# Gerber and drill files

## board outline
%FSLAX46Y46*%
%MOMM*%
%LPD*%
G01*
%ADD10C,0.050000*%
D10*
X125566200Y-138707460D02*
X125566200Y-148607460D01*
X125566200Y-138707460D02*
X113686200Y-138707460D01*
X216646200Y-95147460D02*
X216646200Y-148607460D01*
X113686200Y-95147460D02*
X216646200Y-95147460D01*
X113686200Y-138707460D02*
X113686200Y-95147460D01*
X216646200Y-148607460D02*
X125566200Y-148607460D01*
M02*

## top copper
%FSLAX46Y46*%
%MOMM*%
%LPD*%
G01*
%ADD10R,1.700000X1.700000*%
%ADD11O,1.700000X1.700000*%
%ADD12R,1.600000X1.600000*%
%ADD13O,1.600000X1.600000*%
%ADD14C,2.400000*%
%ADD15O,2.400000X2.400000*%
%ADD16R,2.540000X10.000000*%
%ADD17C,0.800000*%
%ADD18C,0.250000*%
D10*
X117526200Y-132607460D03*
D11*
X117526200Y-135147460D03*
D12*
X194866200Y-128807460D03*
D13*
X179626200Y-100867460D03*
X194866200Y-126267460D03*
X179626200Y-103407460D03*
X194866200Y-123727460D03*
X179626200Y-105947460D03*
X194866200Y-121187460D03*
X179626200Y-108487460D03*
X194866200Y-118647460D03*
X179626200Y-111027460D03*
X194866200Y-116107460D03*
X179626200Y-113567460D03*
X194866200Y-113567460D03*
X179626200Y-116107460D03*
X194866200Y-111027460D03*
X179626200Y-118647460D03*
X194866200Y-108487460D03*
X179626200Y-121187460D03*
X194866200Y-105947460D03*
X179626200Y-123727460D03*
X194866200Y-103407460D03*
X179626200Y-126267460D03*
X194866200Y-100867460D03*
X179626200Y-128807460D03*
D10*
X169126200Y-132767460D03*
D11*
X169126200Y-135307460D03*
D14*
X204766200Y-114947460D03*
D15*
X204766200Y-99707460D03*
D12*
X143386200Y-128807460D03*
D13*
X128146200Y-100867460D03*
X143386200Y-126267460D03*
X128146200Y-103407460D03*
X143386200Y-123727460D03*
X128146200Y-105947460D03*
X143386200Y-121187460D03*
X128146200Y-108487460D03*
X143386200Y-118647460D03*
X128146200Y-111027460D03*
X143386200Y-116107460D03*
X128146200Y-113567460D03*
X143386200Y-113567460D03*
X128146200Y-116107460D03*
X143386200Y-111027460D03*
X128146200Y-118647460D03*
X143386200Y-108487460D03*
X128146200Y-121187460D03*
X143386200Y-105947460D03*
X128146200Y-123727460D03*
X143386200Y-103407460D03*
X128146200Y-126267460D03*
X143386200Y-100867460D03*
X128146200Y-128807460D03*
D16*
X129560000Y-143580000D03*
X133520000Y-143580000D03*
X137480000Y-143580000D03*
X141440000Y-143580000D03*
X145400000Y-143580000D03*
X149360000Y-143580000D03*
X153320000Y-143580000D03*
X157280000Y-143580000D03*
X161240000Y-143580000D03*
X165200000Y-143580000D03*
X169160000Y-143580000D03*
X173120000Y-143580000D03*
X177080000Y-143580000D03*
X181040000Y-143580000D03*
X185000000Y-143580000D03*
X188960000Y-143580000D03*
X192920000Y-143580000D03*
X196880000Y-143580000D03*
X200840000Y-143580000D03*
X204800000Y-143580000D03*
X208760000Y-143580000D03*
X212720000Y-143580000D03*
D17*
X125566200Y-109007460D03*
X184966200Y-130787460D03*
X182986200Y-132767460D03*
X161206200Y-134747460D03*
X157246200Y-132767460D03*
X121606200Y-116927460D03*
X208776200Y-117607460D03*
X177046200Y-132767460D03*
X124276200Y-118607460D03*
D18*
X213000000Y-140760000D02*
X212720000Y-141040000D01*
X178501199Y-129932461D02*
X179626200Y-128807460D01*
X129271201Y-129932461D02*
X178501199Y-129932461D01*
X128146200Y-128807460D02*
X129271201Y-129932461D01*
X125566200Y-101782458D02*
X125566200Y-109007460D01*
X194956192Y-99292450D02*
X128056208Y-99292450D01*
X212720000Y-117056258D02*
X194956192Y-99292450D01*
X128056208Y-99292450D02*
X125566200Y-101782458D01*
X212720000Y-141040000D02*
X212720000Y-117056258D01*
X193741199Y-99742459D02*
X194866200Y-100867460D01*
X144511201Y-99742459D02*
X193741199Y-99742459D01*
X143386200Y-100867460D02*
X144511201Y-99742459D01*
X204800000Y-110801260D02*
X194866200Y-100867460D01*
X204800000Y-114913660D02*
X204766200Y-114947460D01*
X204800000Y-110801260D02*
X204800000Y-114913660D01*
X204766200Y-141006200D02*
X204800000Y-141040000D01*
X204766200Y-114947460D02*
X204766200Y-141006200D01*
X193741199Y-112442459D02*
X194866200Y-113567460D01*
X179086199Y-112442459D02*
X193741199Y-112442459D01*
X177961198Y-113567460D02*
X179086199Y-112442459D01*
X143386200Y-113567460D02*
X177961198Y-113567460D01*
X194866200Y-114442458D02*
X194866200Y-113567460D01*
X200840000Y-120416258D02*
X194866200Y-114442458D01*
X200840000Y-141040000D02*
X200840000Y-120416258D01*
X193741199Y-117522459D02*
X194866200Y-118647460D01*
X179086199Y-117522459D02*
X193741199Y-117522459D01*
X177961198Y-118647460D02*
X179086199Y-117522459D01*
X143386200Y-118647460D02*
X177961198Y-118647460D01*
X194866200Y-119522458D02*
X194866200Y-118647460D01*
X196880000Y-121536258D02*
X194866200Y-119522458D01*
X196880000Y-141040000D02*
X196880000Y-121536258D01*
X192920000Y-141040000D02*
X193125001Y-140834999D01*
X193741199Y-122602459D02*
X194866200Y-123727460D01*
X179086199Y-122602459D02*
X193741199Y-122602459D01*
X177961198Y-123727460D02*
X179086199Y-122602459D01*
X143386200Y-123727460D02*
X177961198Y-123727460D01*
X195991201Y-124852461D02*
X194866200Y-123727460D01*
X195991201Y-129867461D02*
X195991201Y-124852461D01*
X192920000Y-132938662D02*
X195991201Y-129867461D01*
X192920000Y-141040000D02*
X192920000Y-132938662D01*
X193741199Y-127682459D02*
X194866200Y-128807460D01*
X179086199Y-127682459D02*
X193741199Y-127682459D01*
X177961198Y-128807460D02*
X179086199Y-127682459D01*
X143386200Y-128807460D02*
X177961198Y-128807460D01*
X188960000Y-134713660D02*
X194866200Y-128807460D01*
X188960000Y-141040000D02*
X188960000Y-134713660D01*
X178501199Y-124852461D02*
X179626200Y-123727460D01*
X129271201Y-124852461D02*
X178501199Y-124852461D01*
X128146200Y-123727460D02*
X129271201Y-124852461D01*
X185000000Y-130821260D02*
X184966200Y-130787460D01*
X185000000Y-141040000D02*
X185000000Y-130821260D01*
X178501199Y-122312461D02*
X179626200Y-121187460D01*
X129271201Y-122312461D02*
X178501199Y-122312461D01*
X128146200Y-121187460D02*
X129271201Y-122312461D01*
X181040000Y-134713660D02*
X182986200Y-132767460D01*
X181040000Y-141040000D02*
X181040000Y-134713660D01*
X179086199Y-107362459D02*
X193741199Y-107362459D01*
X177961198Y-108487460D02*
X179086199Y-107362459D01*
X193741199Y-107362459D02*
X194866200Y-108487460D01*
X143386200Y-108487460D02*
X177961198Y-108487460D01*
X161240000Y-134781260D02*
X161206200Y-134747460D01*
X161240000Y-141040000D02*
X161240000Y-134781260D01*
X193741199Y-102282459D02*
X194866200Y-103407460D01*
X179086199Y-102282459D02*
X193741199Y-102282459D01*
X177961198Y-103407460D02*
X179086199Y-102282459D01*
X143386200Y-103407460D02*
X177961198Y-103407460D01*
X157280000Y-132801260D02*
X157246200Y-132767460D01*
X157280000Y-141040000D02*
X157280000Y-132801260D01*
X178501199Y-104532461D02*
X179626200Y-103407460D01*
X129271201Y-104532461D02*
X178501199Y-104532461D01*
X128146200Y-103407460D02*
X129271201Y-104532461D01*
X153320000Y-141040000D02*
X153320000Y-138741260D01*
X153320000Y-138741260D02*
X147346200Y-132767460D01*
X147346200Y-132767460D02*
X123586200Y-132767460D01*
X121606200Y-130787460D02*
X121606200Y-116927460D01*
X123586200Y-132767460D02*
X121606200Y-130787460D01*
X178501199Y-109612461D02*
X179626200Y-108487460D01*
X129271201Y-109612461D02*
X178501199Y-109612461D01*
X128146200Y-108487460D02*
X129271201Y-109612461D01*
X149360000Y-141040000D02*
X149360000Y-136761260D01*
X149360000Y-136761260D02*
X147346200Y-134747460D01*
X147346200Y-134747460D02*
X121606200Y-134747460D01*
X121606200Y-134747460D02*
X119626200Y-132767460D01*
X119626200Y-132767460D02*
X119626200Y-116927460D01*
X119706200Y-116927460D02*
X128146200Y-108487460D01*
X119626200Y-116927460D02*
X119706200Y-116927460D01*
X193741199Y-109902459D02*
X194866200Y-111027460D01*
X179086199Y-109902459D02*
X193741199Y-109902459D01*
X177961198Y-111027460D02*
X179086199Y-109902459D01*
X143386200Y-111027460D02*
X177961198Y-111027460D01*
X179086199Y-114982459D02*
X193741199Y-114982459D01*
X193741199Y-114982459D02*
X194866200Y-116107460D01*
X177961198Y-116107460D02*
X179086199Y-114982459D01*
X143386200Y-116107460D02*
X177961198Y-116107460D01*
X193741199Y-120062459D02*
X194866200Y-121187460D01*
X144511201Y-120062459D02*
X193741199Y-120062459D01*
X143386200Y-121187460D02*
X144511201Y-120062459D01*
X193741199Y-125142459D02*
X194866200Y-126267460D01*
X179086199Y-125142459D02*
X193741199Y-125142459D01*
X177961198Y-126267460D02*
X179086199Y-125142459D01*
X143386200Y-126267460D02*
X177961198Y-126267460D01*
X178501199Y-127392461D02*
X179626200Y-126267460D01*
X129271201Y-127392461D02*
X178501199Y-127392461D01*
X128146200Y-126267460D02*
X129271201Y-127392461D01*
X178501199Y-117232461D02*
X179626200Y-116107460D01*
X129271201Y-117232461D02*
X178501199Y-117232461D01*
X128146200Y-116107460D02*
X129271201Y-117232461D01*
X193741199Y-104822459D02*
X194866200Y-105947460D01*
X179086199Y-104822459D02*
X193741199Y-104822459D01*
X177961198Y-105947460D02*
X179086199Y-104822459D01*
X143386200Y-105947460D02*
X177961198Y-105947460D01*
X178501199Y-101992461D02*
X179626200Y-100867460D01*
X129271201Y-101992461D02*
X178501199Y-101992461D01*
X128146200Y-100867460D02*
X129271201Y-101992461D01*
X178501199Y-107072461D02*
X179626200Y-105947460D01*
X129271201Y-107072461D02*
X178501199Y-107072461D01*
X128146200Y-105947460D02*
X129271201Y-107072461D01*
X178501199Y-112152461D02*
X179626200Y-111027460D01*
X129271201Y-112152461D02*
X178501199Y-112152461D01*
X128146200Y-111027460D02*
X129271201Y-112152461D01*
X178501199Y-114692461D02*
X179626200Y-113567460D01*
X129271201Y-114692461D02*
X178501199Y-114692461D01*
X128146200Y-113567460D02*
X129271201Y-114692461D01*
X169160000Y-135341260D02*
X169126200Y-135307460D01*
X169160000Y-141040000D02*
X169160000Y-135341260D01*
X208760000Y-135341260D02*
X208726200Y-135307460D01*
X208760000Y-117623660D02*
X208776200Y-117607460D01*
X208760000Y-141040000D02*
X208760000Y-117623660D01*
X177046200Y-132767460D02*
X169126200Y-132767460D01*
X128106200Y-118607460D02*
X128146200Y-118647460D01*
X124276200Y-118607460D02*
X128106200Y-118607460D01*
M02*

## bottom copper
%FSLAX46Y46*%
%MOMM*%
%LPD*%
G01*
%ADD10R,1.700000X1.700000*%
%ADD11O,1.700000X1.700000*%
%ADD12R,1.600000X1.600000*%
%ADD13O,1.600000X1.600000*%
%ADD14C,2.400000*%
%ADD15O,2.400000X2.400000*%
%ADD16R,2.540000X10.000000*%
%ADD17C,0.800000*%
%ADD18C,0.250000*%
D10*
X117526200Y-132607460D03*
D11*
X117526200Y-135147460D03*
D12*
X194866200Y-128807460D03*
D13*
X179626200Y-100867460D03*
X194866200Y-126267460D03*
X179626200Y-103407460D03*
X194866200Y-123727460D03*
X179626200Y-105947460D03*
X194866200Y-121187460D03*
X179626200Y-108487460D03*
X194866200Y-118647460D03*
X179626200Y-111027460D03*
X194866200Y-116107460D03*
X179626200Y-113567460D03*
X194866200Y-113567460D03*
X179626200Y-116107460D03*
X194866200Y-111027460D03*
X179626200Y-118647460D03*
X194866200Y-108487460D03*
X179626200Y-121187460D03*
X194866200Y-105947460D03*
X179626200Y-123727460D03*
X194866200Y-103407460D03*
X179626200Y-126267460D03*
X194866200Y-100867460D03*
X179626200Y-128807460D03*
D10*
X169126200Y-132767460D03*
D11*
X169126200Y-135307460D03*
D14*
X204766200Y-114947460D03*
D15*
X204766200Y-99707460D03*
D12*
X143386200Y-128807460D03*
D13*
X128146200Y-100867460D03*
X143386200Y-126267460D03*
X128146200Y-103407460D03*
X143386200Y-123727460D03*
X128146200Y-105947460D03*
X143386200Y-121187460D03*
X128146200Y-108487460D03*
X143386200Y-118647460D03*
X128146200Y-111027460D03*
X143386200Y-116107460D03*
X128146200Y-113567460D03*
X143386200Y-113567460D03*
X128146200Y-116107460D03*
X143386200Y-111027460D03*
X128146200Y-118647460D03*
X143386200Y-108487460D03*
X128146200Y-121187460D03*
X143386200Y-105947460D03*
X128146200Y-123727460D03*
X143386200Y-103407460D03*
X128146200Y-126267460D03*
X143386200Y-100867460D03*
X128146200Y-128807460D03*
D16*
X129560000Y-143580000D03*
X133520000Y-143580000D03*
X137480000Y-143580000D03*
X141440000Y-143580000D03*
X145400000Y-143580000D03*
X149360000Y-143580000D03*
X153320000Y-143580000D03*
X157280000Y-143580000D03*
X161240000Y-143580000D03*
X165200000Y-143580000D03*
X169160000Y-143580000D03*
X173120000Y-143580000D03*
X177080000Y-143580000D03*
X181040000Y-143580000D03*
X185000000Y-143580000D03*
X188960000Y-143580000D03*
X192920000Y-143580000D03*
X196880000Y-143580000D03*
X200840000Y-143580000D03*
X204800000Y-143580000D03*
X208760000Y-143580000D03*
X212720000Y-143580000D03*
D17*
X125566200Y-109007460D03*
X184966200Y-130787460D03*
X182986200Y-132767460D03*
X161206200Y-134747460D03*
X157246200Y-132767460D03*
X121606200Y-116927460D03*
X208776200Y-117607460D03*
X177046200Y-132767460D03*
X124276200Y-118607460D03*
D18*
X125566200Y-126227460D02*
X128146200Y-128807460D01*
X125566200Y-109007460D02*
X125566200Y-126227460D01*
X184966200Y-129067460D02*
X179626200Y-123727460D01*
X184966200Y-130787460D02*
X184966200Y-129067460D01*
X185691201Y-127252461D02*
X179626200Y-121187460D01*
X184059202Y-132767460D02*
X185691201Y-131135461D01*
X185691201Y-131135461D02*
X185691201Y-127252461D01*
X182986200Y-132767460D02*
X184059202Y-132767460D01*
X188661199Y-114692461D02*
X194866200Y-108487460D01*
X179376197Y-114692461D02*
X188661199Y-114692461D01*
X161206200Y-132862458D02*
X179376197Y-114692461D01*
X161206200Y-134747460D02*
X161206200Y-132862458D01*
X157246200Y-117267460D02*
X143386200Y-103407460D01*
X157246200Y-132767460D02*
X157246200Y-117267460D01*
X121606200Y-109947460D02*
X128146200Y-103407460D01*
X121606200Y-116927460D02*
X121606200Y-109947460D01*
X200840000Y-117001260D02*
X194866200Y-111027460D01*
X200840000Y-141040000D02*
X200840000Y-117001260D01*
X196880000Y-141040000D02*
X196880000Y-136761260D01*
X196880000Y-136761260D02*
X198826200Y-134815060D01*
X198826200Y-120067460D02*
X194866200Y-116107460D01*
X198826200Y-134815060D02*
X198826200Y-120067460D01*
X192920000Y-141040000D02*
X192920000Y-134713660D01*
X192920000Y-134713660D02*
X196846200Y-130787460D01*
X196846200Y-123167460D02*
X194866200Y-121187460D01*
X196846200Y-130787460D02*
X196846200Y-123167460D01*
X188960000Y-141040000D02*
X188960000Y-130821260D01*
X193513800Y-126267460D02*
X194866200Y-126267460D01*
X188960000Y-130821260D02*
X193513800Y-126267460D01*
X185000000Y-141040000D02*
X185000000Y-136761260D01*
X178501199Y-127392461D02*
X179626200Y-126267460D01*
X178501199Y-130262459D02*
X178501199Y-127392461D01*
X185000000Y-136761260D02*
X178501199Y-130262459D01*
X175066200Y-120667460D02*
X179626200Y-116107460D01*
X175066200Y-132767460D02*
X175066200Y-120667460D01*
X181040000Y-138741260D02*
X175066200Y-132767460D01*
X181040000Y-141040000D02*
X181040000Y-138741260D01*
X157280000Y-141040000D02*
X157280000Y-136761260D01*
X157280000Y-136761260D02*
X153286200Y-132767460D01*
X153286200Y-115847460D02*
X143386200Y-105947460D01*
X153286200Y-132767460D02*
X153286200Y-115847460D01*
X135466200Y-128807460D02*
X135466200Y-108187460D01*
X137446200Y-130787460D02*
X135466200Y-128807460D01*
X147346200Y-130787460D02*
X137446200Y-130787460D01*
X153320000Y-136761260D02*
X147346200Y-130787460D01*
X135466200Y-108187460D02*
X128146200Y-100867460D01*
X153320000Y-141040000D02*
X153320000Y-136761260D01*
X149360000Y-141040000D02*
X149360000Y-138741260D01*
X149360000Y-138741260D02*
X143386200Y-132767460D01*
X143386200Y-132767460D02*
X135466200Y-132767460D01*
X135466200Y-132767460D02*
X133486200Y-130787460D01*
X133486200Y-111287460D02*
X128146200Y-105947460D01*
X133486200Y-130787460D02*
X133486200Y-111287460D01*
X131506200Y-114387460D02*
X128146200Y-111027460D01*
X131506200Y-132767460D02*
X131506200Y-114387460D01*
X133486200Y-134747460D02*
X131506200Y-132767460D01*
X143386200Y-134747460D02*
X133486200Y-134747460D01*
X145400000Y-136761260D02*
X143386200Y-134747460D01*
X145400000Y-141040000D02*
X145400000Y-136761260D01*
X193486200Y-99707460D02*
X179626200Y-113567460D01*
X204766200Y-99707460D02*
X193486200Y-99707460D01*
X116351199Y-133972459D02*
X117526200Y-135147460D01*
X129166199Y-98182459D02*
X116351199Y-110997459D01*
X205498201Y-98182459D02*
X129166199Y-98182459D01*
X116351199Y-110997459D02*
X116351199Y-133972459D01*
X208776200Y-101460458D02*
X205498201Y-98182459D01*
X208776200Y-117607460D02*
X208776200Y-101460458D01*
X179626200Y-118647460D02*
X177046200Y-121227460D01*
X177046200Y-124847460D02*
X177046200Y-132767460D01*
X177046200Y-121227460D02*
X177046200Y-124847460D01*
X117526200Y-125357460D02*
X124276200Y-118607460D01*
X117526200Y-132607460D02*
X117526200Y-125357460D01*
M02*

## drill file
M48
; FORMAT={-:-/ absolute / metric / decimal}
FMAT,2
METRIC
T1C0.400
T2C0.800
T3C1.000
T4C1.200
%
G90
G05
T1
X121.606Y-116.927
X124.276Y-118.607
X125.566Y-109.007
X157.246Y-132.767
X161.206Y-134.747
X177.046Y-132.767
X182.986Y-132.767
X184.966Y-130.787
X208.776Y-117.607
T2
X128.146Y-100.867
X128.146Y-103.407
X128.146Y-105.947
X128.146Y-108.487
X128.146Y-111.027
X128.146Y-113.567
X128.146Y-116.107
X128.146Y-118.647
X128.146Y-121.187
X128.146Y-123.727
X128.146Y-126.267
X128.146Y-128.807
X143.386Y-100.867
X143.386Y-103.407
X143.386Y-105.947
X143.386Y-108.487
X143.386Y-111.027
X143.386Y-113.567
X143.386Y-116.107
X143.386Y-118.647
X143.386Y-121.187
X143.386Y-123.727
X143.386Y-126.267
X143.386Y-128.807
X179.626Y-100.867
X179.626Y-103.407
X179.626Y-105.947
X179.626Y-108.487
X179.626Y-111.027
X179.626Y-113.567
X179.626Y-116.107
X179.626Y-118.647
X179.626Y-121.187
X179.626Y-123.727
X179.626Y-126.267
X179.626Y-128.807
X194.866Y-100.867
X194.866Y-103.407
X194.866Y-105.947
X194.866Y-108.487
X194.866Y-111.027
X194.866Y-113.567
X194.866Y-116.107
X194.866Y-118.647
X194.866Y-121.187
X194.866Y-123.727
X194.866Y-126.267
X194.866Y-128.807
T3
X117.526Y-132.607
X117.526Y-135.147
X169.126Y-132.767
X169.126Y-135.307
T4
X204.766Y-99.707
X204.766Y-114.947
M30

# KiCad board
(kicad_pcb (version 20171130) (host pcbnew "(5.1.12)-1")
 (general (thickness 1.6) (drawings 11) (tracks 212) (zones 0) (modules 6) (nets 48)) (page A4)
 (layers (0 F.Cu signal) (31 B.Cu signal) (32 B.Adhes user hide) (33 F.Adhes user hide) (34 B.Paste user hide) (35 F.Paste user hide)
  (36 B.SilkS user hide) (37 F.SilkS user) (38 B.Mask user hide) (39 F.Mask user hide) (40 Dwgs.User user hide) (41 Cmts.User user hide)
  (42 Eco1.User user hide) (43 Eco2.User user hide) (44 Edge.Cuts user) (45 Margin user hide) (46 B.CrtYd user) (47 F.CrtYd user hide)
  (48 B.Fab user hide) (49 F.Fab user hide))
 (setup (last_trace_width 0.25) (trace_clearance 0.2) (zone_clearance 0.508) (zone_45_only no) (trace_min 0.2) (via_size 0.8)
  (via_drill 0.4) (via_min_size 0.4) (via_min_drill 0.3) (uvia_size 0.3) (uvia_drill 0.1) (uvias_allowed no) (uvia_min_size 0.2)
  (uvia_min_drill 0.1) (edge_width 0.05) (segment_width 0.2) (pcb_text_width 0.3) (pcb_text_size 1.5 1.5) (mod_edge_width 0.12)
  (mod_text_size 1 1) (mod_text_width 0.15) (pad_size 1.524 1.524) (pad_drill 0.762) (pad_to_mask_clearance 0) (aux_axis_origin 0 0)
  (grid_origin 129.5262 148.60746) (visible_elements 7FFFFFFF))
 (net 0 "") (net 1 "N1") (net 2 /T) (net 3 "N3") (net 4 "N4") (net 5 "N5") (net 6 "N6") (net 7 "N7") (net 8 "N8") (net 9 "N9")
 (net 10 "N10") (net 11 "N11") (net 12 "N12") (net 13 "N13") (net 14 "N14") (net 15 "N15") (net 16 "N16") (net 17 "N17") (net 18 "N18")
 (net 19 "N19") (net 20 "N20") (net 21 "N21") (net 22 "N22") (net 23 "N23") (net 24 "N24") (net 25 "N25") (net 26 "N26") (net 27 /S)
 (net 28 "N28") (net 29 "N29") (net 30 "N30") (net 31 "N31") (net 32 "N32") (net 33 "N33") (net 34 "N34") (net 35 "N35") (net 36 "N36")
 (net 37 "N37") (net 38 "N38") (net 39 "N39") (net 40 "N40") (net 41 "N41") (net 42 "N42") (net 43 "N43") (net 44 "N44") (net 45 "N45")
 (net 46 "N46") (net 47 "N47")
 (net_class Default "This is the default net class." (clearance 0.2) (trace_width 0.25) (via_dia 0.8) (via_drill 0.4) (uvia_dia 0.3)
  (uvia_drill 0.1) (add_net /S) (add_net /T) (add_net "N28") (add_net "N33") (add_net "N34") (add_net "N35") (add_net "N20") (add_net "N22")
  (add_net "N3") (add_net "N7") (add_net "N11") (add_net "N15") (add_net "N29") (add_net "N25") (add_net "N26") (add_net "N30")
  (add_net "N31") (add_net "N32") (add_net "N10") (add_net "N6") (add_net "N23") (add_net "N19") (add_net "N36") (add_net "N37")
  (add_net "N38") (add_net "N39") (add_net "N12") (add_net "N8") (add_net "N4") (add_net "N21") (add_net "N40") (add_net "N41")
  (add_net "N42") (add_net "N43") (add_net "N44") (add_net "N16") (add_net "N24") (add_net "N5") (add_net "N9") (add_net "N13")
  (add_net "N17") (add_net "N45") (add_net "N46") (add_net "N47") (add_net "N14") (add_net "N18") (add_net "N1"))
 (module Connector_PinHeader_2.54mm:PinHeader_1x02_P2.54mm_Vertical (layer F.Cu) (at 117.5262 132.60746)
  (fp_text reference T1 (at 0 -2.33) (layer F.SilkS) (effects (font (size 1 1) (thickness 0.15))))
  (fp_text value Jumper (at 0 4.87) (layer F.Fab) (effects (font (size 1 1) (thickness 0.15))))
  (pad 1 thru_hole rect (at 0 0) (size 1.7 1.7) (drill 1) (layers *.Cu *.Mask) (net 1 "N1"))
  (pad 2 thru_hole oval (at 0 2.54) (size 1.7 1.7) (drill 1) (layers *.Cu *.Mask) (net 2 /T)))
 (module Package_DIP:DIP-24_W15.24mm (layer F.Cu) (at 194.8662 128.80746 180)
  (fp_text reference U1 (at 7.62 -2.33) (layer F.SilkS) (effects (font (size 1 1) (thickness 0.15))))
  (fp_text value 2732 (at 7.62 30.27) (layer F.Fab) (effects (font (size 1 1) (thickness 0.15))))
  (pad 1 thru_hole rect (at 0 0 180) (size 1.6 1.6) (drill 0.8) (layers *.Cu *.Mask) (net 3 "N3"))
  (pad 13 thru_hole oval (at 15.24 27.94 180) (size 1.6 1.6) (drill 0.8) (layers *.Cu *.Mask) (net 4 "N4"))
  (pad 2 thru_hole oval (at 0 2.54 180) (size 1.6 1.6) (drill 0.8) (layers *.Cu *.Mask) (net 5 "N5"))
  (pad 14 thru_hole oval (at 15.24 25.4 180) (size 1.6 1.6) (drill 0.8) (layers *.Cu *.Mask) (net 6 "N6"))
  (pad 3 thru_hole oval (at 0 5.08 180) (size 1.6 1.6) (drill 0.8) (layers *.Cu *.Mask) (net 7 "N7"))
  (pad 15 thru_hole oval (at 15.24 22.86 180) (size 1.6 1.6) (drill 0.8) (layers *.Cu *.Mask) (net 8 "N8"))
  (pad 4 thru_hole oval (at 0 7.62 180) (size 1.6 1.6) (drill 0.8) (layers *.Cu *.Mask) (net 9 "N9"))
  (pad 16 thru_hole oval (at 15.24 20.32 180) (size 1.6 1.6) (drill 0.8) (layers *.Cu *.Mask) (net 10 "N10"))
  (pad 5 thru_hole oval (at 0 10.16 180) (size 1.6 1.6) (drill 0.8) (layers *.Cu *.Mask) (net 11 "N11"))
  (pad 17 thru_hole oval (at 15.24 17.78 180) (size 1.6 1.6) (drill 0.8) (layers *.Cu *.Mask) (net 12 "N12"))
  (pad 6 thru_hole oval (at 0 12.7 180) (size 1.6 1.6) (drill 0.8) (layers *.Cu *.Mask) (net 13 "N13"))
  (pad 18 thru_hole oval (at 15.24 15.24 180) (size 1.6 1.6) (drill 0.8) (layers *.Cu *.Mask) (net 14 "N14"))
  (pad 7 thru_hole oval (at 0 15.24 180) (size 1.6 1.6) (drill 0.8) (layers *.Cu *.Mask) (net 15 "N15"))
  (pad 19 thru_hole oval (at 15.24 12.7 180) (size 1.6 1.6) (drill 0.8) (layers *.Cu *.Mask) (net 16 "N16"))
  (pad 8 thru_hole oval (at 0 17.78 180) (size 1.6 1.6) (drill 0.8) (layers *.Cu *.Mask) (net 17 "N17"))
  (pad 20 thru_hole oval (at 15.24 10.16 180) (size 1.6 1.6) (drill 0.8) (layers *.Cu *.Mask) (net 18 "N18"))
  (pad 9 thru_hole oval (at 0 20.32 180) (size 1.6 1.6) (drill 0.8) (layers *.Cu *.Mask) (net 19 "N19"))
  (pad 21 thru_hole oval (at 15.24 7.62 180) (size 1.6 1.6) (drill 0.8) (layers *.Cu *.Mask) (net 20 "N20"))
  (pad 10 thru_hole oval (at 0 22.86 180) (size 1.6 1.6) (drill 0.8) (layers *.Cu *.Mask) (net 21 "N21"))
  (pad 22 thru_hole oval (at 15.24 5.08 180) (size 1.6 1.6) (drill 0.8) (layers *.Cu *.Mask) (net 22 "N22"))
  (pad 11 thru_hole oval (at 0 25.4 180) (size 1.6 1.6) (drill 0.8) (layers *.Cu *.Mask) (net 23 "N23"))
  (pad 23 thru_hole oval (at 15.24 2.54 180) (size 1.6 1.6) (drill 0.8) (layers *.Cu *.Mask) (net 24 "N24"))
  (pad 12 thru_hole oval (at 0 27.94 180) (size 1.6 1.6) (drill 0.8) (layers *.Cu *.Mask) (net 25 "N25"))
  (pad 24 thru_hole oval (at 15.24 0 180) (size 1.6 1.6) (drill 0.8) (layers *.Cu *.Mask) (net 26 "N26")))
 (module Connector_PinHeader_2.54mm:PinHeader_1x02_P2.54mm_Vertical (layer F.Cu) (at 169.1262 132.76746)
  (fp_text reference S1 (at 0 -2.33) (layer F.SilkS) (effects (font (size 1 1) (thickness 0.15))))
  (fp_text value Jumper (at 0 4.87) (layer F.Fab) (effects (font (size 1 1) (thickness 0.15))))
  (pad 1 thru_hole rect (at 0 0) (size 1.7 1.7) (drill 1) (layers *.Cu *.Mask) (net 18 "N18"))
  (pad 2 thru_hole oval (at 0 2.54) (size 1.7 1.7) (drill 1) (layers *.Cu *.Mask) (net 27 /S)))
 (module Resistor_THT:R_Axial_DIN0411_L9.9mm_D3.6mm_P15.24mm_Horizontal (layer F.Cu) (at 204.7662 114.94746 90)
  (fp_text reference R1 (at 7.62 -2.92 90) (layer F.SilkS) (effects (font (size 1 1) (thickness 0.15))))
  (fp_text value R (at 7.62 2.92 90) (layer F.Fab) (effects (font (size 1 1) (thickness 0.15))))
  (pad 1 thru_hole circle (at 0 0 90) (size 2.4 2.4) (drill 1.2) (layers *.Cu *.Mask) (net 25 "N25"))
  (pad 2 thru_hole oval (at 15.24 0 90) (size 2.4 2.4) (drill 1.2) (layers *.Cu *.Mask) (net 14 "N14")))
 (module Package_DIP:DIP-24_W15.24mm (layer F.Cu) (at 143.3862 128.80746 180)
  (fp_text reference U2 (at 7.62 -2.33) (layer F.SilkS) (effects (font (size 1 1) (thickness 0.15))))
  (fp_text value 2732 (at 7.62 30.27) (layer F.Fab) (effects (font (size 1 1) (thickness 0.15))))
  (pad 1 thru_hole rect (at 0 0 180) (size 1.6 1.6) (drill 0.8) (layers *.Cu *.Mask) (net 3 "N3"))
  (pad 13 thru_hole oval (at 15.24 27.94 180) (size 1.6 1.6) (drill 0.8) (layers *.Cu *.Mask) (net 4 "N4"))
  (pad 2 thru_hole oval (at 0 2.54 180) (size 1.6 1.6) (drill 0.8) (layers *.Cu *.Mask) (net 5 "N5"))
  (pad 14 thru_hole oval (at 15.24 25.4 180) (size 1.6 1.6) (drill 0.8) (layers *.Cu *.Mask) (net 6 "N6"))
  (pad 3 thru_hole oval (at 0 5.08 180) (size 1.6 1.6) (drill 0.8) (layers *.Cu *.Mask) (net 7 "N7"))
  (pad 15 thru_hole oval (at 15.24 22.86 180) (size 1.6 1.6) (drill 0.8) (layers *.Cu *.Mask) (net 8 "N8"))
  (pad 4 thru_hole oval (at 0 7.62 180) (size 1.6 1.6) (drill 0.8) (layers *.Cu *.Mask) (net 9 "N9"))
  (pad 16 thru_hole oval (at 15.24 20.32 180) (size 1.6 1.6) (drill 0.8) (layers *.Cu *.Mask) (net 10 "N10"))
  (pad 5 thru_hole oval (at 0 10.16 180) (size 1.6 1.6) (drill 0.8) (layers *.Cu *.Mask) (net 11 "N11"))
  (pad 17 thru_hole oval (at 15.24 17.78 180) (size 1.6 1.6) (drill 0.8) (layers *.Cu *.Mask) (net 12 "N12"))
  (pad 6 thru_hole oval (at 0 12.7 180) (size 1.6 1.6) (drill 0.8) (layers *.Cu *.Mask) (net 13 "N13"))
  (pad 18 thru_hole oval (at 15.24 15.24 180) (size 1.6 1.6) (drill 0.8) (layers *.Cu *.Mask) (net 14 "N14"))
  (pad 7 thru_hole oval (at 0 15.24 180) (size 1.6 1.6) (drill 0.8) (layers *.Cu *.Mask) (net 15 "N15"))
  (pad 19 thru_hole oval (at 15.24 12.7 180) (size 1.6 1.6) (drill 0.8) (layers *.Cu *.Mask) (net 16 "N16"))
  (pad 8 thru_hole oval (at 0 17.78 180) (size 1.6 1.6) (drill 0.8) (layers *.Cu *.Mask) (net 17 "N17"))
  (pad 20 thru_hole oval (at 15.24 10.16 180) (size 1.6 1.6) (drill 0.8) (layers *.Cu *.Mask) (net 1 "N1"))
  (pad 9 thru_hole oval (at 0 20.32 180) (size 1.6 1.6) (drill 0.8) (layers *.Cu *.Mask) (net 19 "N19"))
  (pad 21 thru_hole oval (at 15.24 7.62 180) (size 1.6 1.6) (drill 0.8) (layers *.Cu *.Mask) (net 20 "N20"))
  (pad 10 thru_hole oval (at 0 22.86 180) (size 1.6 1.6) (drill 0.8) (layers *.Cu *.Mask) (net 21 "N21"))
  (pad 22 thru_hole oval (at 15.24 5.08 180) (size 1.6 1.6) (drill 0.8) (layers *.Cu *.Mask) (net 22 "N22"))
  (pad 11 thru_hole oval (at 0 25.4 180) (size 1.6 1.6) (drill 0.8) (layers *.Cu *.Mask) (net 23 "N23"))
  (pad 23 thru_hole oval (at 15.24 2.54 180) (size 1.6 1.6) (drill 0.8) (layers *.Cu *.Mask) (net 24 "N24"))
  (pad 12 thru_hole oval (at 0 27.94 180) (size 1.6 1.6) (drill 0.8) (layers *.Cu *.Mask) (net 25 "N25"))
  (pad 24 thru_hole oval (at 15.24 0 180) (size 1.6 1.6) (drill 0.8) (layers *.Cu *.Mask) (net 26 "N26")))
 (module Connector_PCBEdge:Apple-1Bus (layer F.Cu) (at 185 145)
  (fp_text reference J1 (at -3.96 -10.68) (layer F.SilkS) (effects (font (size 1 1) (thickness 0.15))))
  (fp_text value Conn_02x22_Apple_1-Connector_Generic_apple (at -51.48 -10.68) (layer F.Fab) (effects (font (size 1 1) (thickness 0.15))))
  (pad 1 connect rect (at -55.44 -3.96) (size 2.54 10) (drill (offset 0 2.54)) (layers F.Cu F.Mask) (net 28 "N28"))
  (pad 2 connect rect (at -51.48 -3.96) (size 2.54 10) (drill (offset 0 2.54)) (layers F.Cu F.Mask) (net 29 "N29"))
  (pad 3 connect rect (at -47.52 -3.96) (size 2.54 10) (drill (offset 0 2.54)) (layers F.Cu F.Mask) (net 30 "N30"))
  (pad 4 connect rect (at -43.56 -3.96) (size 2.54 10) (drill (offset 0 2.54)) (layers F.Cu F.Mask) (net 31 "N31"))
  (pad 5 connect rect (at -39.6 -3.96) (size 2.54 10) (drill (offset 0 2.54)) (layers F.Cu F.Mask) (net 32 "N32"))
  (pad 6 connect rect (at -35.64 -3.96) (size 2.54 10) (drill (offset 0 2.54)) (layers F.Cu F.Mask) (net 10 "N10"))
  (pad 7 connect rect (at -31.68 -3.96) (size 2.54 10) (drill (offset 0 2.54)) (layers F.Cu F.Mask) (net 6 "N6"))
  (pad 8 connect rect (at -27.72 -3.96) (size 2.54 10) (drill (offset 0 2.54)) (layers F.Cu F.Mask) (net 23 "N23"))
  (pad 9 connect rect (at -23.76 -3.96) (size 2.54 10) (drill (offset 0 2.54)) (layers F.Cu F.Mask) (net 19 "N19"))
  (pad 10 connect rect (at -19.8 -3.96) (size 2.54 10) (drill (offset 0 2.54)) (layers F.Cu F.Mask) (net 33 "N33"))
  (pad 11 connect rect (at -15.84 -3.96) (size 2.54 10) (drill (offset 0 2.54)) (layers F.Cu F.Mask) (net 27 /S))
  (pad 12 connect rect (at -11.88 -3.96) (size 2.54 10) (drill (offset 0 2.54)) (layers F.Cu F.Mask) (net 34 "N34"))
  (pad 13 connect rect (at -7.92 -3.96) (size 2.54 10) (drill (offset 0 2.54)) (layers F.Cu F.Mask) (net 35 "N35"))
  (pad 14 connect rect (at -3.96 -3.96) (size 2.54 10) (drill (offset 0 2.54)) (layers F.Cu F.Mask) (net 20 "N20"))
  (pad 15 connect rect (at 0 -3.96) (size 2.54 10) (drill (offset 0 2.54)) (layers F.Cu F.Mask) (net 22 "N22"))
  (pad 16 connect rect (at 3.96 -3.96) (size 2.54 10) (drill (offset 0 2.54)) (layers F.Cu F.Mask) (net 3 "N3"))
  (pad 17 connect rect (at 7.92 -3.96) (size 2.54 10) (drill (offset 0 2.54)) (layers F.Cu F.Mask) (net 7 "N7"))
  (pad 18 connect rect (at 11.88 -3.96) (size 2.54 10) (drill (offset 0 2.54)) (layers F.Cu F.Mask) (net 11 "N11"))
  (pad 19 connect rect (at 15.84 -3.96) (size 2.54 10) (drill (offset 0 2.54)) (layers F.Cu F.Mask) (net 15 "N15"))
  (pad 20 connect rect (at 19.8 -3.96) (size 2.54 10) (drill (offset 0 2.54)) (layers F.Cu F.Mask) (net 25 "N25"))
  (pad 21 connect rect (at 23.76 -3.96) (size 2.54 10) (drill (offset 0 2.54)) (layers F.Cu F.Mask) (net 2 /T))
  (pad 22 connect rect (at 27.72 -3.96) (size 2.54 10) (drill (offset 0 2.54)) (layers F.Cu F.Mask) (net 26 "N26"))
  (pad A connect rect (at -55.44 -3.96) (size 2.54 10) (drill (offset 0 2.54)) (layers B.Cu B.Mask) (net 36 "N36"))
  (pad B connect rect (at -51.48 -3.96) (size 2.54 10) (drill (offset 0 2.54)) (layers B.Cu B.Mask) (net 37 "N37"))
  (pad C connect rect (at -47.52 -3.96) (size 2.54 10) (drill (offset 0 2.54)) (layers B.Cu B.Mask) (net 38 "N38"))
  (pad D connect rect (at -43.56 -3.96) (size 2.54 10) (drill (offset 0 2.54)) (layers B.Cu B.Mask) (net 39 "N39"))
  (pad E connect rect (at -39.6 -3.96) (size 2.54 10) (drill (offset 0 2.54)) (layers B.Cu B.Mask) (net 12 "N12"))
  (pad F connect rect (at -35.64 -3.96) (size 2.54 10) (drill (offset 0 2.54)) (layers B.Cu B.Mask) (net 8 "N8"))
  (pad H connect rect (at -31.68 -3.96) (size 2.54 10) (drill (offset 0 2.54)) (layers B.Cu B.Mask) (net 4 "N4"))
  (pad J connect rect (at -27.72 -3.96) (size 2.54 10) (drill (offset 0 2.54)) (layers B.Cu B.Mask) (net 21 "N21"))
  (pad K connect rect (at -23.76 -3.96) (size 2.54 10) (drill (offset 0 2.54)) (layers B.Cu B.Mask) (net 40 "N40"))
  (pad L connect rect (at -19.8 -3.96) (size 2.54 10) (drill (offset 0 2.54)) (layers B.Cu B.Mask) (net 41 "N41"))
  (pad M connect rect (at -15.84 -3.96) (size 2.54 10) (drill (offset 0 2.54)) (layers B.Cu B.Mask) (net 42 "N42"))
  (pad N connect rect (at -11.88 -3.96) (size 2.54 10) (drill (offset 0 2.54)) (layers B.Cu B.Mask) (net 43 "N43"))
  (pad P connect rect (at -7.92 -3.96) (size 2.54 10) (drill (offset 0 2.54)) (layers B.Cu B.Mask) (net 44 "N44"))
  (pad R connect rect (at -3.96 -3.96) (size 2.54 10) (drill (offset 0 2.54)) (layers B.Cu B.Mask) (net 16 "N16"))
  (pad S connect rect (at 0 -3.96) (size 2.54 10) (drill (offset 0 2.54)) (layers B.Cu B.Mask) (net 24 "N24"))
  (pad T connect rect (at 3.96 -3.96) (size 2.54 10) (drill (offset 0 2.54)) (layers B.Cu B.Mask) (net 5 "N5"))
  (pad U connect rect (at 7.92 -3.96) (size 2.54 10) (drill (offset 0 2.54)) (layers B.Cu B.Mask) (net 9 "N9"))
  (pad V connect rect (at 11.88 -3.96) (size 2.54 10) (drill (offset 0 2.54)) (layers B.Cu B.Mask) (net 13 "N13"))
  (pad W connect rect (at 15.84 -3.96) (size 2.54 10) (drill (offset 0 2.54)) (layers B.Cu B.Mask) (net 17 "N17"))
  (pad X connect rect (at 19.8 -3.96) (size 2.54 10) (drill (offset 0 2.54)) (layers B.Cu B.Mask) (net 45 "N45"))
  (pad Y connect rect (at 23.76 -3.96) (size 2.54 10) (drill (offset 0 2.54)) (layers B.Cu B.Mask) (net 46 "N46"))
  (pad Z connect rect (at 27.72 -3.96) (size 2.54 10) (drill (offset 0 2.54)) (layers B.Cu B.Mask) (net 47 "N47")))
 (gr_line (start 125.5662 138.70746) (end 125.5662 148.60746) (layer Edge.Cuts) (width 0.05))
 (gr_line (start 125.5662 138.70746) (end 113.6862 138.70746) (layer Edge.Cuts) (width 0.05))
 (gr_line (start 216.6462 95.14746) (end 216.6462 148.60746) (layer Edge.Cuts) (width 0.05))
 (gr_line (start 113.6862 95.14746) (end 216.6462 95.14746) (layer Edge.Cuts) (width 0.05))
 (gr_line (start 113.6862 138.70746) (end 113.6862 95.14746) (layer Edge.Cuts) (width 0.05))
 (gr_line (start 216.6462 148.60746) (end 125.5662 148.60746) (layer Edge.Cuts) (width 0.05))
 (segment (start 213 140.76) (end 212.72 141.04) (width 0.25) (layer F.Cu) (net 26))
 (segment (start 178.501199 129.932461) (end 179.6262 128.80746) (width 0.25) (layer F.Cu) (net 26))
 (segment (start 129.271201 129.932461) (end 178.501199 129.932461) (width 0.25) (layer F.Cu) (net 26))
 (segment (start 128.1462 128.80746) (end 129.271201 129.932461) (width 0.25) (layer F.Cu) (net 26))
 (via (at 125.5662 109.00746) (size 0.8) (drill 0.4) (layers F.Cu B.Cu) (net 26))
 (segment (start 125.5662 101.782458) (end 125.5662 109.00746) (width 0.25) (layer F.Cu) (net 26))
 (segment (start 194.956192 99.29245) (end 128.056208 99.29245) (width 0.25) (layer F.Cu) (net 26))
 (segment (start 212.72 117.056258) (end 194.956192 99.29245) (width 0.25) (layer F.Cu) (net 26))
 (segment (start 128.056208 99.29245) (end 125.5662 101.782458) (width 0.25) (layer F.Cu) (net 26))
 (segment (start 212.72 141.04) (end 212.72 117.056258) (width 0.25) (layer F.Cu) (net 26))
 (segment (start 125.5662 126.22746) (end 128.1462 128.80746) (width 0.25) (layer B.Cu) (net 26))
 (segment (start 125.5662 109.00746) (end 125.5662 126.22746) (width 0.25) (layer B.Cu) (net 26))
 (segment (start 193.741199 99.742459) (end 194.8662 100.86746) (width 0.25) (layer F.Cu) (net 25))
 (segment (start 144.511201 99.742459) (end 193.741199 99.742459) (width 0.25) (layer F.Cu) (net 25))
 (segment (start 143.3862 100.86746) (end 144.511201 99.742459) (width 0.25) (layer F.Cu) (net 25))
 (segment (start 204.8 110.80126) (end 194.8662 100.86746) (width 0.25) (layer F.Cu) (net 25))
 (segment (start 204.8 114.91366) (end 204.7662 114.94746) (width 0.25) (layer F.Cu) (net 25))
 (segment (start 204.8 110.80126) (end 204.8 114.91366) (width 0.25) (layer F.Cu) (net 25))
 (segment (start 204.7662 141.0062) (end 204.8 141.04) (width 0.25) (layer F.Cu) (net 25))
 (segment (start 204.7662 114.94746) (end 204.7662 141.0062) (width 0.25) (layer F.Cu) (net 25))
 (segment (start 193.741199 112.442459) (end 194.8662 113.56746) (width 0.25) (layer F.Cu) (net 15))
 (segment (start 179.086199 112.442459) (end 193.741199 112.442459) (width 0.25) (layer F.Cu) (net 15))
 (segment (start 177.961198 113.56746) (end 179.086199 112.442459) (width 0.25) (layer F.Cu) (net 15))
 (segment (start 143.3862 113.56746) (end 177.961198 113.56746) (width 0.25) (layer F.Cu) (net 15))
 (segment (start 194.8662 114.442458) (end 194.8662 113.56746) (width 0.25) (layer F.Cu) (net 15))
 (segment (start 200.84 120.416258) (end 194.8662 114.442458) (width 0.25) (layer F.Cu) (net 15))
 (segment (start 200.84 141.04) (end 200.84 120.416258) (width 0.25) (layer F.Cu) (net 15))
 (segment (start 193.741199 117.522459) (end 194.8662 118.64746) (width 0.25) (layer F.Cu) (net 11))
 (segment (start 179.086199 117.522459) (end 193.741199 117.522459) (width 0.25) (layer F.Cu) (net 11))
 (segment (start 177.961198 118.64746) (end 179.086199 117.522459) (width 0.25) (layer F.Cu) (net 11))
 (segment (start 143.3862 118.64746) (end 177.961198 118.64746) (width 0.25) (layer F.Cu) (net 11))
 (segment (start 194.8662 119.522458) (end 194.8662 118.64746) (width 0.25) (layer F.Cu) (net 11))
 (segment (start 196.88 121.536258) (end 194.8662 119.522458) (width 0.25) (layer F.Cu) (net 11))
 (segment (start 196.88 141.04) (end 196.88 121.536258) (width 0.25) (layer F.Cu) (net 11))
 (segment (start 192.92 141.04) (end 193.125001 140.834999) (width 0.25) (layer F.Cu) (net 7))
 (segment (start 193.741199 122.602459) (end 194.8662 123.72746) (width 0.25) (layer F.Cu) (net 7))
 (segment (start 179.086199 122.602459) (end 193.741199 122.602459) (width 0.25) (layer F.Cu) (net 7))
 (segment (start 177.961198 123.72746) (end 179.086199 122.602459) (width 0.25) (layer F.Cu) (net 7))
 (segment (start 143.3862 123.72746) (end 177.961198 123.72746) (width 0.25) (layer F.Cu) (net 7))
 (segment (start 195.991201 124.852461) (end 194.8662 123.72746) (width 0.25) (layer F.Cu) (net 7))
 (segment (start 195.991201 129.867461) (end 195.991201 124.852461) (width 0.25) (layer F.Cu) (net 7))
 (segment (start 192.92 132.938662) (end 195.991201 129.867461) (width 0.25) (layer F.Cu) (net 7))
 (segment (start 192.92 141.04) (end 192.92 132.938662) (width 0.25) (layer F.Cu) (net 7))
 (segment (start 193.741199 127.682459) (end 194.8662 128.80746) (width 0.25) (layer F.Cu) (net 3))
 (segment (start 179.086199 127.682459) (end 193.741199 127.682459) (width 0.25) (layer F.Cu) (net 3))
 (segment (start 177.961198 128.80746) (end 179.086199 127.682459) (width 0.25) (layer F.Cu) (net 3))
 (segment (start 143.3862 128.80746) (end 177.961198 128.80746) (width 0.25) (layer F.Cu) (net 3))
 (segment (start 188.96 134.71366) (end 194.8662 128.80746) (width 0.25) (layer F.Cu) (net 3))
 (segment (start 188.96 141.04) (end 188.96 134.71366) (width 0.25) (layer F.Cu) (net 3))
 (segment (start 178.501199 124.852461) (end 179.6262 123.72746) (width 0.25) (layer F.Cu) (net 22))
 (segment (start 129.271201 124.852461) (end 178.501199 124.852461) (width 0.25) (layer F.Cu) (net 22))
 (segment (start 128.1462 123.72746) (end 129.271201 124.852461) (width 0.25) (layer F.Cu) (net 22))
 (via (at 184.9662 130.78746) (size 0.8) (drill 0.4) (layers F.Cu B.Cu) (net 22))
 (segment (start 185 130.82126) (end 184.9662 130.78746) (width 0.25) (layer F.Cu) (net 22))
 (segment (start 185 141.04) (end 185 130.82126) (width 0.25) (layer F.Cu) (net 22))
 (segment (start 184.9662 129.06746) (end 179.6262 123.72746) (width 0.25) (layer B.Cu) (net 22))
 (segment (start 184.9662 130.78746) (end 184.9662 129.06746) (width 0.25) (layer B.Cu) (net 22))
 (segment (start 178.501199 122.312461) (end 179.6262 121.18746) (width 0.25) (layer F.Cu) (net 20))
 (segment (start 129.271201 122.312461) (end 178.501199 122.312461) (width 0.25) (layer F.Cu) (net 20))
 (segment (start 128.1462 121.18746) (end 129.271201 122.312461) (width 0.25) (layer F.Cu) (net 20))
 (via (at 182.9862 132.76746) (size 0.8) (drill 0.4) (layers F.Cu B.Cu) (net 20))
 (segment (start 181.04 134.71366) (end 182.9862 132.76746) (width 0.25) (layer F.Cu) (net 20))
 (segment (start 181.04 141.04) (end 181.04 134.71366) (width 0.25) (layer F.Cu) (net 20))
 (segment (start 185.691201 127.252461) (end 179.6262 121.18746) (width 0.25) (layer B.Cu) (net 20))
 (segment (start 184.059202 132.76746) (end 185.691201 131.135461) (width 0.25) (layer B.Cu) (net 20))
 (segment (start 185.691201 131.135461) (end 185.691201 127.252461) (width 0.25) (layer B.Cu) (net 20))
 (segment (start 182.9862 132.76746) (end 184.059202 132.76746) (width 0.25) (layer B.Cu) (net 20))
 (segment (start 179.086199 107.362459) (end 193.741199 107.362459) (width 0.25) (layer F.Cu) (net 19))
 (segment (start 177.961198 108.48746) (end 179.086199 107.362459) (width 0.25) (layer F.Cu) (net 19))
 (segment (start 193.741199 107.362459) (end 194.8662 108.48746) (width 0.25) (layer F.Cu) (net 19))
 (segment (start 143.3862 108.48746) (end 177.961198 108.48746) (width 0.25) (layer F.Cu) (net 19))
 (via (at 161.2062 134.74746) (size 0.8) (drill 0.4) (layers F.Cu B.Cu) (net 19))
 (segment (start 161.24 134.78126) (end 161.2062 134.74746) (width 0.25) (layer F.Cu) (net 19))
 (segment (start 161.24 141.04) (end 161.24 134.78126) (width 0.25) (layer F.Cu) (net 19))
 (segment (start 188.661199 114.692461) (end 194.8662 108.48746) (width 0.25) (layer B.Cu) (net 19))
 (segment (start 179.376197 114.692461) (end 188.661199 114.692461) (width 0.25) (layer B.Cu) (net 19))
 (segment (start 161.2062 132.862458) (end 179.376197 114.692461) (width 0.25) (layer B.Cu) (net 19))
 (segment (start 161.2062 134.74746) (end 161.2062 132.862458) (width 0.25) (layer B.Cu) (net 19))
 (segment (start 193.741199 102.282459) (end 194.8662 103.40746) (width 0.25) (layer F.Cu) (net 23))
 (segment (start 179.086199 102.282459) (end 193.741199 102.282459) (width 0.25) (layer F.Cu) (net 23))
 (segment (start 177.961198 103.40746) (end 179.086199 102.282459) (width 0.25) (layer F.Cu) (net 23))
 (segment (start 143.3862 103.40746) (end 177.961198 103.40746) (width 0.25) (layer F.Cu) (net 23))
 (via (at 157.2462 132.76746) (size 0.8) (drill 0.4) (layers F.Cu B.Cu) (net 23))
 (segment (start 157.28 132.80126) (end 157.2462 132.76746) (width 0.25) (layer F.Cu) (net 23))
 (segment (start 157.28 141.04) (end 157.28 132.80126) (width 0.25) (layer F.Cu) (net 23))
 (segment (start 157.2462 117.26746) (end 143.3862 103.40746) (width 0.25) (layer B.Cu) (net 23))
 (segment (start 157.2462 132.76746) (end 157.2462 117.26746) (width 0.25) (layer B.Cu) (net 23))
 (segment (start 178.501199 104.532461) (end 179.6262 103.40746) (width 0.25) (layer F.Cu) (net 6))
 (segment (start 129.271201 104.532461) (end 178.501199 104.532461) (width 0.25) (layer F.Cu) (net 6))
 (segment (start 128.1462 103.40746) (end 129.271201 104.532461) (width 0.25) (layer F.Cu) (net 6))
 (segment (start 153.32 141.04) (end 153.32 138.74126) (width 0.25) (layer F.Cu) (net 6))
 (segment (start 153.32 138.74126) (end 147.3462 132.76746) (width 0.25) (layer F.Cu) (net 6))
 (segment (start 147.3462 132.76746) (end 123.5862 132.76746) (width 0.25) (layer F.Cu) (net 6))
 (via (at 121.6062 116.92746) (size 0.8) (drill 0.4) (layers F.Cu B.Cu) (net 6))
 (segment (start 121.6062 130.78746) (end 121.6062 116.92746) (width 0.25) (layer F.Cu) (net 6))
 (segment (start 123.5862 132.76746) (end 121.6062 130.78746) (width 0.25) (layer F.Cu) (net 6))
 (segment (start 121.6062 109.94746) (end 128.1462 103.40746) (width 0.25) (layer B.Cu) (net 6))
 (segment (start 121.6062 116.92746) (end 121.6062 109.94746) (width 0.25) (layer B.Cu) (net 6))
 (segment (start 178.501199 109.612461) (end 179.6262 108.48746) (width 0.25) (layer F.Cu) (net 10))
 (segment (start 129.271201 109.612461) (end 178.501199 109.612461) (width 0.25) (layer F.Cu) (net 10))
 (segment (start 128.1462 108.48746) (end 129.271201 109.612461) (width 0.25) (layer F.Cu) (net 10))
 (segment (start 149.36 141.04) (end 149.36 136.76126) (width 0.25) (layer F.Cu) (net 10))
 (segment (start 149.36 136.76126) (end 147.3462 134.74746) (width 0.25) (layer F.Cu) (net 10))
 (segment (start 147.3462 134.74746) (end 121.6062 134.74746) (width 0.25) (layer F.Cu) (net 10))
 (segment (start 121.6062 134.74746) (end 119.6262 132.76746) (width 0.25) (layer F.Cu) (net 10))
 (segment (start 119.6262 132.76746) (end 119.6262 116.92746) (width 0.25) (layer F.Cu) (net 10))
 (segment (start 119.7062 116.92746) (end 128.1462 108.48746) (width 0.25) (layer F.Cu) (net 10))
 (segment (start 119.6262 116.92746) (end 119.7062 116.92746) (width 0.25) (layer F.Cu) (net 10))
 (segment (start 193.741199 109.902459) (end 194.8662 111.02746) (width 0.25) (layer F.Cu) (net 17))
 (segment (start 179.086199 109.902459) (end 193.741199 109.902459) (width 0.25) (layer F.Cu) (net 17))
 (segment (start 177.961198 111.02746) (end 179.086199 109.902459) (width 0.25) (layer F.Cu) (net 17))
 (segment (start 143.3862 111.02746) (end 177.961198 111.02746) (width 0.25) (layer F.Cu) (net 17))
 (segment (start 200.84 117.00126) (end 194.8662 111.02746) (width 0.25) (layer B.Cu) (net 17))
 (segment (start 200.84 141.04) (end 200.84 117.00126) (width 0.25) (layer B.Cu) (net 17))
 (segment (start 179.086199 114.982459) (end 193.741199 114.982459) (width 0.25) (layer F.Cu) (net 13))
 (segment (start 193.741199 114.982459) (end 194.8662 116.10746) (width 0.25) (layer F.Cu) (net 13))
 (segment (start 177.961198 116.10746) (end 179.086199 114.982459) (width 0.25) (layer F.Cu) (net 13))
 (segment (start 143.3862 116.10746) (end 177.961198 116.10746) (width 0.25) (layer F.Cu) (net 13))
 (segment (start 196.88 141.04) (end 196.88 136.76126) (width 0.25) (layer B.Cu) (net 13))
 (segment (start 196.88 136.76126) (end 198.8262 134.81506) (width 0.25) (layer B.Cu) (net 13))
 (segment (start 198.8262 120.06746) (end 194.8662 116.10746) (width 0.25) (layer B.Cu) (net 13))
 (segment (start 198.8262 134.81506) (end 198.8262 120.06746) (width 0.25) (layer B.Cu) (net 13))
 (segment (start 193.741199 120.062459) (end 194.8662 121.18746) (width 0.25) (layer F.Cu) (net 9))
 (segment (start 144.511201 120.062459) (end 193.741199 120.062459) (width 0.25) (layer F.Cu) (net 9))
 (segment (start 143.3862 121.18746) (end 144.511201 120.062459) (width 0.25) (layer F.Cu) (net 9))
 (segment (start 192.92 141.04) (end 192.92 134.71366) (width 0.25) (layer B.Cu) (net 9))
 (segment (start 192.92 134.71366) (end 196.8462 130.78746) (width 0.25) (layer B.Cu) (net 9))
 (segment (start 196.8462 123.16746) (end 194.8662 121.18746) (width 0.25) (layer B.Cu) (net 9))
 (segment (start 196.8462 130.78746) (end 196.8462 123.16746) (width 0.25) (layer B.Cu) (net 9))
 (segment (start 193.741199 125.142459) (end 194.8662 126.26746) (width 0.25) (layer F.Cu) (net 5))
 (segment (start 179.086199 125.142459) (end 193.741199 125.142459) (width 0.25) (layer F.Cu) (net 5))
 (segment (start 177.961198 126.26746) (end 179.086199 125.142459) (width 0.25) (layer F.Cu) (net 5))
 (segment (start 143.3862 126.26746) (end 177.961198 126.26746) (width 0.25) (layer F.Cu) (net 5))
 (segment (start 188.96 141.04) (end 188.96 130.82126) (width 0.25) (layer B.Cu) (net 5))
 (segment (start 193.5138 126.26746) (end 194.8662 126.26746) (width 0.25) (layer B.Cu) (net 5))
 (segment (start 188.96 130.82126) (end 193.5138 126.26746) (width 0.25) (layer B.Cu) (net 5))
 (segment (start 178.501199 127.392461) (end 179.6262 126.26746) (width 0.25) (layer F.Cu) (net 24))
 (segment (start 129.271201 127.392461) (end 178.501199 127.392461) (width 0.25) (layer F.Cu) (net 24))
 (segment (start 128.1462 126.26746) (end 129.271201 127.392461) (width 0.25) (layer F.Cu) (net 24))
 (segment (start 185 141.04) (end 185 136.76126) (width 0.25) (layer B.Cu) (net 24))
 (segment (start 178.501199 127.392461) (end 179.6262 126.26746) (width 0.25) (layer B.Cu) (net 24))
 (segment (start 178.501199 130.262459) (end 178.501199 127.392461) (width 0.25) (layer B.Cu) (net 24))
 (segment (start 185 136.76126) (end 178.501199 130.262459) (width 0.25) (layer B.Cu) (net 24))
 (segment (start 178.501199 117.232461) (end 179.6262 116.10746) (width 0.25) (layer F.Cu) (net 16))
 (segment (start 129.271201 117.232461) (end 178.501199 117.232461) (width 0.25) (layer F.Cu) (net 16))
 (segment (start 128.1462 116.10746) (end 129.271201 117.232461) (width 0.25) (layer F.Cu) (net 16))
 (segment (start 175.0662 120.66746) (end 179.6262 116.10746) (width 0.25) (layer B.Cu) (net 16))
 (segment (start 175.0662 132.76746) (end 175.0662 120.66746) (width 0.25) (layer B.Cu) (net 16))
 (segment (start 181.04 138.74126) (end 175.0662 132.76746) (width 0.25) (layer B.Cu) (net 16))
 (segment (start 181.04 141.04) (end 181.04 138.74126) (width 0.25) (layer B.Cu) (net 16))
 (segment (start 193.741199 104.822459) (end 194.8662 105.94746) (width 0.25) (layer F.Cu) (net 21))
 (segment (start 179.086199 104.822459) (end 193.741199 104.822459) (width 0.25) (layer F.Cu) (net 21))
 (segment (start 177.961198 105.94746) (end 179.086199 104.822459) (width 0.25) (layer F.Cu) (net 21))
 (segment (start 143.3862 105.94746) (end 177.961198 105.94746) (width 0.25) (layer F.Cu) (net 21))
 (segment (start 157.28 141.04) (end 157.28 136.76126) (width 0.25) (layer B.Cu) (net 21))
 (segment (start 157.28 136.76126) (end 153.2862 132.76746) (width 0.25) (layer B.Cu) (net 21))
 (segment (start 153.2862 115.84746) (end 143.3862 105.94746) (width 0.25) (layer B.Cu) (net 21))
 (segment (start 153.2862 132.76746) (end 153.2862 115.84746) (width 0.25) (layer B.Cu) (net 21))
 (segment (start 178.501199 101.992461) (end 179.6262 100.86746) (width 0.25) (layer F.Cu) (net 4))
 (segment (start 129.271201 101.992461) (end 178.501199 101.992461) (width 0.25) (layer F.Cu) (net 4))
 (segment (start 128.1462 100.86746) (end 129.271201 101.992461) (width 0.25) (layer F.Cu) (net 4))
 (segment (start 135.4662 128.80746) (end 135.4662 108.18746) (width 0.25) (layer B.Cu) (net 4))
 (segment (start 137.4462 130.78746) (end 135.4662 128.80746) (width 0.25) (layer B.Cu) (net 4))
 (segment (start 147.3462 130.78746) (end 137.4462 130.78746) (width 0.25) (layer B.Cu) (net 4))
 (segment (start 153.32 136.76126) (end 147.3462 130.78746) (width 0.25) (layer B.Cu) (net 4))
 (segment (start 135.4662 108.18746) (end 128.1462 100.86746) (width 0.25) (layer B.Cu) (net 4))
 (segment (start 153.32 141.04) (end 153.32 136.76126) (width 0.25) (layer B.Cu) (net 4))
 (segment (start 178.501199 107.072461) (end 179.6262 105.94746) (width 0.25) (layer F.Cu) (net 8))
 (segment (start 129.271201 107.072461) (end 178.501199 107.072461) (width 0.25) (layer F.Cu) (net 8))
 (segment (start 128.1462 105.94746) (end 129.271201 107.072461) (width 0.25) (layer F.Cu) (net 8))
 (segment (start 149.36 141.04) (end 149.36 138.74126) (width 0.25) (layer B.Cu) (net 8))
 (segment (start 149.36 138.74126) (end 143.3862 132.76746) (width 0.25) (layer B.Cu) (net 8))
 (segment (start 143.3862 132.76746) (end 135.4662 132.76746) (width 0.25) (layer B.Cu) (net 8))
 (segment (start 135.4662 132.76746) (end 133.4862 130.78746) (width 0.25) (layer B.Cu) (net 8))
 (segment (start 133.4862 111.28746) (end 128.1462 105.94746) (width 0.25) (layer B.Cu) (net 8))
 (segment (start 133.4862 130.78746) (end 133.4862 111.28746) (width 0.25) (layer B.Cu) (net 8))
 (segment (start 178.501199 112.152461) (end 179.6262 111.02746) (width 0.25) (layer F.Cu) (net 12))
 (segment (start 129.271201 112.152461) (end 178.501199 112.152461) (width 0.25) (layer F.Cu) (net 12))
 (segment (start 128.1462 111.02746) (end 129.271201 112.152461) (width 0.25) (layer F.Cu) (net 12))
 (segment (start 131.5062 114.38746) (end 128.1462 111.02746) (width 0.25) (layer B.Cu) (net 12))
 (segment (start 131.5062 132.76746) (end 131.5062 114.38746) (width 0.25) (layer B.Cu) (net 12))
 (segment (start 133.4862 134.74746) (end 131.5062 132.76746) (width 0.25) (layer B.Cu) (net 12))
 (segment (start 143.3862 134.74746) (end 133.4862 134.74746) (width 0.25) (layer B.Cu) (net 12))
 (segment (start 145.4 136.76126) (end 143.3862 134.74746) (width 0.25) (layer B.Cu) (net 12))
 (segment (start 145.4 141.04) (end 145.4 136.76126) (width 0.25) (layer B.Cu) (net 12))
 (segment (start 178.501199 114.692461) (end 179.6262 113.56746) (width 0.25) (layer F.Cu) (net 14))
 (segment (start 129.271201 114.692461) (end 178.501199 114.692461) (width 0.25) (layer F.Cu) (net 14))
 (segment (start 128.1462 113.56746) (end 129.271201 114.692461) (width 0.25) (layer F.Cu) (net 14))
 (segment (start 193.4862 99.70746) (end 179.6262 113.56746) (width 0.25) (layer B.Cu) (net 14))
 (segment (start 204.7662 99.70746) (end 193.4862 99.70746) (width 0.25) (layer B.Cu) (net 14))
 (segment (start 169.16 135.34126) (end 169.1262 135.30746) (width 0.25) (layer F.Cu) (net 27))
 (segment (start 169.16 141.04) (end 169.16 135.34126) (width 0.25) (layer F.Cu) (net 27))
 (segment (start 208.76 135.34126) (end 208.7262 135.30746) (width 0.25) (layer F.Cu) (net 2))
 (via (at 208.7762 117.60746) (size 0.8) (drill 0.4) (layers F.Cu B.Cu) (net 2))
 (segment (start 208.76 117.62366) (end 208.7762 117.60746) (width 0.25) (layer F.Cu) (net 2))
 (segment (start 208.76 141.04) (end 208.76 117.62366) (width 0.25) (layer F.Cu) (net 2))
 (segment (start 116.351199 133.972459) (end 117.5262 135.14746) (width 0.25) (layer B.Cu) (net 2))
 (segment (start 129.166199 98.182459) (end 116.351199 110.997459) (width 0.25) (layer B.Cu) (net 2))
 (segment (start 205.498201 98.182459) (end 129.166199 98.182459) (width 0.25) (layer B.Cu) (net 2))
 (segment (start 116.351199 110.997459) (end 116.351199 133.972459) (width 0.25) (layer B.Cu) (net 2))
 (segment (start 208.7762 101.460458) (end 205.498201 98.182459) (width 0.25) (layer B.Cu) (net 2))
 (segment (start 208.7762 117.60746) (end 208.7762 101.460458) (width 0.25) (layer B.Cu) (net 2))
 (segment (start 179.6262 118.64746) (end 177.0462 121.22746) (width 0.25) (layer B.Cu) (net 18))
 (via (at 177.0462 132.76746) (size 0.8) (drill 0.4) (layers F.Cu B.Cu) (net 18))
 (segment (start 177.0462 124.84746) (end 177.0462 132.76746) (width 0.25) (layer B.Cu) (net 18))
 (segment (start 177.0462 121.22746) (end 177.0462 124.84746) (width 0.25) (layer B.Cu) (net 18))
 (segment (start 177.0462 132.76746) (end 169.1262 132.76746) (width 0.25) (layer F.Cu) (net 18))
 (via (at 124.2762 118.60746) (size 0.8) (drill 0.4) (layers F.Cu B.Cu) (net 1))
 (segment (start 117.5262 125.35746) (end 124.2762 118.60746) (width 0.25) (layer B.Cu) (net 1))
 (segment (start 117.5262 132.60746) (end 117.5262 125.35746) (width 0.25) (layer B.Cu) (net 1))
 (segment (start 128.1062 118.60746) (end 128.1462 118.64746) (width 0.25) (layer F.Cu) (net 1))
 (segment (start 124.2762 118.60746) (end 128.1062 118.60746) (width 0.25) (layer F.Cu) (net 1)))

